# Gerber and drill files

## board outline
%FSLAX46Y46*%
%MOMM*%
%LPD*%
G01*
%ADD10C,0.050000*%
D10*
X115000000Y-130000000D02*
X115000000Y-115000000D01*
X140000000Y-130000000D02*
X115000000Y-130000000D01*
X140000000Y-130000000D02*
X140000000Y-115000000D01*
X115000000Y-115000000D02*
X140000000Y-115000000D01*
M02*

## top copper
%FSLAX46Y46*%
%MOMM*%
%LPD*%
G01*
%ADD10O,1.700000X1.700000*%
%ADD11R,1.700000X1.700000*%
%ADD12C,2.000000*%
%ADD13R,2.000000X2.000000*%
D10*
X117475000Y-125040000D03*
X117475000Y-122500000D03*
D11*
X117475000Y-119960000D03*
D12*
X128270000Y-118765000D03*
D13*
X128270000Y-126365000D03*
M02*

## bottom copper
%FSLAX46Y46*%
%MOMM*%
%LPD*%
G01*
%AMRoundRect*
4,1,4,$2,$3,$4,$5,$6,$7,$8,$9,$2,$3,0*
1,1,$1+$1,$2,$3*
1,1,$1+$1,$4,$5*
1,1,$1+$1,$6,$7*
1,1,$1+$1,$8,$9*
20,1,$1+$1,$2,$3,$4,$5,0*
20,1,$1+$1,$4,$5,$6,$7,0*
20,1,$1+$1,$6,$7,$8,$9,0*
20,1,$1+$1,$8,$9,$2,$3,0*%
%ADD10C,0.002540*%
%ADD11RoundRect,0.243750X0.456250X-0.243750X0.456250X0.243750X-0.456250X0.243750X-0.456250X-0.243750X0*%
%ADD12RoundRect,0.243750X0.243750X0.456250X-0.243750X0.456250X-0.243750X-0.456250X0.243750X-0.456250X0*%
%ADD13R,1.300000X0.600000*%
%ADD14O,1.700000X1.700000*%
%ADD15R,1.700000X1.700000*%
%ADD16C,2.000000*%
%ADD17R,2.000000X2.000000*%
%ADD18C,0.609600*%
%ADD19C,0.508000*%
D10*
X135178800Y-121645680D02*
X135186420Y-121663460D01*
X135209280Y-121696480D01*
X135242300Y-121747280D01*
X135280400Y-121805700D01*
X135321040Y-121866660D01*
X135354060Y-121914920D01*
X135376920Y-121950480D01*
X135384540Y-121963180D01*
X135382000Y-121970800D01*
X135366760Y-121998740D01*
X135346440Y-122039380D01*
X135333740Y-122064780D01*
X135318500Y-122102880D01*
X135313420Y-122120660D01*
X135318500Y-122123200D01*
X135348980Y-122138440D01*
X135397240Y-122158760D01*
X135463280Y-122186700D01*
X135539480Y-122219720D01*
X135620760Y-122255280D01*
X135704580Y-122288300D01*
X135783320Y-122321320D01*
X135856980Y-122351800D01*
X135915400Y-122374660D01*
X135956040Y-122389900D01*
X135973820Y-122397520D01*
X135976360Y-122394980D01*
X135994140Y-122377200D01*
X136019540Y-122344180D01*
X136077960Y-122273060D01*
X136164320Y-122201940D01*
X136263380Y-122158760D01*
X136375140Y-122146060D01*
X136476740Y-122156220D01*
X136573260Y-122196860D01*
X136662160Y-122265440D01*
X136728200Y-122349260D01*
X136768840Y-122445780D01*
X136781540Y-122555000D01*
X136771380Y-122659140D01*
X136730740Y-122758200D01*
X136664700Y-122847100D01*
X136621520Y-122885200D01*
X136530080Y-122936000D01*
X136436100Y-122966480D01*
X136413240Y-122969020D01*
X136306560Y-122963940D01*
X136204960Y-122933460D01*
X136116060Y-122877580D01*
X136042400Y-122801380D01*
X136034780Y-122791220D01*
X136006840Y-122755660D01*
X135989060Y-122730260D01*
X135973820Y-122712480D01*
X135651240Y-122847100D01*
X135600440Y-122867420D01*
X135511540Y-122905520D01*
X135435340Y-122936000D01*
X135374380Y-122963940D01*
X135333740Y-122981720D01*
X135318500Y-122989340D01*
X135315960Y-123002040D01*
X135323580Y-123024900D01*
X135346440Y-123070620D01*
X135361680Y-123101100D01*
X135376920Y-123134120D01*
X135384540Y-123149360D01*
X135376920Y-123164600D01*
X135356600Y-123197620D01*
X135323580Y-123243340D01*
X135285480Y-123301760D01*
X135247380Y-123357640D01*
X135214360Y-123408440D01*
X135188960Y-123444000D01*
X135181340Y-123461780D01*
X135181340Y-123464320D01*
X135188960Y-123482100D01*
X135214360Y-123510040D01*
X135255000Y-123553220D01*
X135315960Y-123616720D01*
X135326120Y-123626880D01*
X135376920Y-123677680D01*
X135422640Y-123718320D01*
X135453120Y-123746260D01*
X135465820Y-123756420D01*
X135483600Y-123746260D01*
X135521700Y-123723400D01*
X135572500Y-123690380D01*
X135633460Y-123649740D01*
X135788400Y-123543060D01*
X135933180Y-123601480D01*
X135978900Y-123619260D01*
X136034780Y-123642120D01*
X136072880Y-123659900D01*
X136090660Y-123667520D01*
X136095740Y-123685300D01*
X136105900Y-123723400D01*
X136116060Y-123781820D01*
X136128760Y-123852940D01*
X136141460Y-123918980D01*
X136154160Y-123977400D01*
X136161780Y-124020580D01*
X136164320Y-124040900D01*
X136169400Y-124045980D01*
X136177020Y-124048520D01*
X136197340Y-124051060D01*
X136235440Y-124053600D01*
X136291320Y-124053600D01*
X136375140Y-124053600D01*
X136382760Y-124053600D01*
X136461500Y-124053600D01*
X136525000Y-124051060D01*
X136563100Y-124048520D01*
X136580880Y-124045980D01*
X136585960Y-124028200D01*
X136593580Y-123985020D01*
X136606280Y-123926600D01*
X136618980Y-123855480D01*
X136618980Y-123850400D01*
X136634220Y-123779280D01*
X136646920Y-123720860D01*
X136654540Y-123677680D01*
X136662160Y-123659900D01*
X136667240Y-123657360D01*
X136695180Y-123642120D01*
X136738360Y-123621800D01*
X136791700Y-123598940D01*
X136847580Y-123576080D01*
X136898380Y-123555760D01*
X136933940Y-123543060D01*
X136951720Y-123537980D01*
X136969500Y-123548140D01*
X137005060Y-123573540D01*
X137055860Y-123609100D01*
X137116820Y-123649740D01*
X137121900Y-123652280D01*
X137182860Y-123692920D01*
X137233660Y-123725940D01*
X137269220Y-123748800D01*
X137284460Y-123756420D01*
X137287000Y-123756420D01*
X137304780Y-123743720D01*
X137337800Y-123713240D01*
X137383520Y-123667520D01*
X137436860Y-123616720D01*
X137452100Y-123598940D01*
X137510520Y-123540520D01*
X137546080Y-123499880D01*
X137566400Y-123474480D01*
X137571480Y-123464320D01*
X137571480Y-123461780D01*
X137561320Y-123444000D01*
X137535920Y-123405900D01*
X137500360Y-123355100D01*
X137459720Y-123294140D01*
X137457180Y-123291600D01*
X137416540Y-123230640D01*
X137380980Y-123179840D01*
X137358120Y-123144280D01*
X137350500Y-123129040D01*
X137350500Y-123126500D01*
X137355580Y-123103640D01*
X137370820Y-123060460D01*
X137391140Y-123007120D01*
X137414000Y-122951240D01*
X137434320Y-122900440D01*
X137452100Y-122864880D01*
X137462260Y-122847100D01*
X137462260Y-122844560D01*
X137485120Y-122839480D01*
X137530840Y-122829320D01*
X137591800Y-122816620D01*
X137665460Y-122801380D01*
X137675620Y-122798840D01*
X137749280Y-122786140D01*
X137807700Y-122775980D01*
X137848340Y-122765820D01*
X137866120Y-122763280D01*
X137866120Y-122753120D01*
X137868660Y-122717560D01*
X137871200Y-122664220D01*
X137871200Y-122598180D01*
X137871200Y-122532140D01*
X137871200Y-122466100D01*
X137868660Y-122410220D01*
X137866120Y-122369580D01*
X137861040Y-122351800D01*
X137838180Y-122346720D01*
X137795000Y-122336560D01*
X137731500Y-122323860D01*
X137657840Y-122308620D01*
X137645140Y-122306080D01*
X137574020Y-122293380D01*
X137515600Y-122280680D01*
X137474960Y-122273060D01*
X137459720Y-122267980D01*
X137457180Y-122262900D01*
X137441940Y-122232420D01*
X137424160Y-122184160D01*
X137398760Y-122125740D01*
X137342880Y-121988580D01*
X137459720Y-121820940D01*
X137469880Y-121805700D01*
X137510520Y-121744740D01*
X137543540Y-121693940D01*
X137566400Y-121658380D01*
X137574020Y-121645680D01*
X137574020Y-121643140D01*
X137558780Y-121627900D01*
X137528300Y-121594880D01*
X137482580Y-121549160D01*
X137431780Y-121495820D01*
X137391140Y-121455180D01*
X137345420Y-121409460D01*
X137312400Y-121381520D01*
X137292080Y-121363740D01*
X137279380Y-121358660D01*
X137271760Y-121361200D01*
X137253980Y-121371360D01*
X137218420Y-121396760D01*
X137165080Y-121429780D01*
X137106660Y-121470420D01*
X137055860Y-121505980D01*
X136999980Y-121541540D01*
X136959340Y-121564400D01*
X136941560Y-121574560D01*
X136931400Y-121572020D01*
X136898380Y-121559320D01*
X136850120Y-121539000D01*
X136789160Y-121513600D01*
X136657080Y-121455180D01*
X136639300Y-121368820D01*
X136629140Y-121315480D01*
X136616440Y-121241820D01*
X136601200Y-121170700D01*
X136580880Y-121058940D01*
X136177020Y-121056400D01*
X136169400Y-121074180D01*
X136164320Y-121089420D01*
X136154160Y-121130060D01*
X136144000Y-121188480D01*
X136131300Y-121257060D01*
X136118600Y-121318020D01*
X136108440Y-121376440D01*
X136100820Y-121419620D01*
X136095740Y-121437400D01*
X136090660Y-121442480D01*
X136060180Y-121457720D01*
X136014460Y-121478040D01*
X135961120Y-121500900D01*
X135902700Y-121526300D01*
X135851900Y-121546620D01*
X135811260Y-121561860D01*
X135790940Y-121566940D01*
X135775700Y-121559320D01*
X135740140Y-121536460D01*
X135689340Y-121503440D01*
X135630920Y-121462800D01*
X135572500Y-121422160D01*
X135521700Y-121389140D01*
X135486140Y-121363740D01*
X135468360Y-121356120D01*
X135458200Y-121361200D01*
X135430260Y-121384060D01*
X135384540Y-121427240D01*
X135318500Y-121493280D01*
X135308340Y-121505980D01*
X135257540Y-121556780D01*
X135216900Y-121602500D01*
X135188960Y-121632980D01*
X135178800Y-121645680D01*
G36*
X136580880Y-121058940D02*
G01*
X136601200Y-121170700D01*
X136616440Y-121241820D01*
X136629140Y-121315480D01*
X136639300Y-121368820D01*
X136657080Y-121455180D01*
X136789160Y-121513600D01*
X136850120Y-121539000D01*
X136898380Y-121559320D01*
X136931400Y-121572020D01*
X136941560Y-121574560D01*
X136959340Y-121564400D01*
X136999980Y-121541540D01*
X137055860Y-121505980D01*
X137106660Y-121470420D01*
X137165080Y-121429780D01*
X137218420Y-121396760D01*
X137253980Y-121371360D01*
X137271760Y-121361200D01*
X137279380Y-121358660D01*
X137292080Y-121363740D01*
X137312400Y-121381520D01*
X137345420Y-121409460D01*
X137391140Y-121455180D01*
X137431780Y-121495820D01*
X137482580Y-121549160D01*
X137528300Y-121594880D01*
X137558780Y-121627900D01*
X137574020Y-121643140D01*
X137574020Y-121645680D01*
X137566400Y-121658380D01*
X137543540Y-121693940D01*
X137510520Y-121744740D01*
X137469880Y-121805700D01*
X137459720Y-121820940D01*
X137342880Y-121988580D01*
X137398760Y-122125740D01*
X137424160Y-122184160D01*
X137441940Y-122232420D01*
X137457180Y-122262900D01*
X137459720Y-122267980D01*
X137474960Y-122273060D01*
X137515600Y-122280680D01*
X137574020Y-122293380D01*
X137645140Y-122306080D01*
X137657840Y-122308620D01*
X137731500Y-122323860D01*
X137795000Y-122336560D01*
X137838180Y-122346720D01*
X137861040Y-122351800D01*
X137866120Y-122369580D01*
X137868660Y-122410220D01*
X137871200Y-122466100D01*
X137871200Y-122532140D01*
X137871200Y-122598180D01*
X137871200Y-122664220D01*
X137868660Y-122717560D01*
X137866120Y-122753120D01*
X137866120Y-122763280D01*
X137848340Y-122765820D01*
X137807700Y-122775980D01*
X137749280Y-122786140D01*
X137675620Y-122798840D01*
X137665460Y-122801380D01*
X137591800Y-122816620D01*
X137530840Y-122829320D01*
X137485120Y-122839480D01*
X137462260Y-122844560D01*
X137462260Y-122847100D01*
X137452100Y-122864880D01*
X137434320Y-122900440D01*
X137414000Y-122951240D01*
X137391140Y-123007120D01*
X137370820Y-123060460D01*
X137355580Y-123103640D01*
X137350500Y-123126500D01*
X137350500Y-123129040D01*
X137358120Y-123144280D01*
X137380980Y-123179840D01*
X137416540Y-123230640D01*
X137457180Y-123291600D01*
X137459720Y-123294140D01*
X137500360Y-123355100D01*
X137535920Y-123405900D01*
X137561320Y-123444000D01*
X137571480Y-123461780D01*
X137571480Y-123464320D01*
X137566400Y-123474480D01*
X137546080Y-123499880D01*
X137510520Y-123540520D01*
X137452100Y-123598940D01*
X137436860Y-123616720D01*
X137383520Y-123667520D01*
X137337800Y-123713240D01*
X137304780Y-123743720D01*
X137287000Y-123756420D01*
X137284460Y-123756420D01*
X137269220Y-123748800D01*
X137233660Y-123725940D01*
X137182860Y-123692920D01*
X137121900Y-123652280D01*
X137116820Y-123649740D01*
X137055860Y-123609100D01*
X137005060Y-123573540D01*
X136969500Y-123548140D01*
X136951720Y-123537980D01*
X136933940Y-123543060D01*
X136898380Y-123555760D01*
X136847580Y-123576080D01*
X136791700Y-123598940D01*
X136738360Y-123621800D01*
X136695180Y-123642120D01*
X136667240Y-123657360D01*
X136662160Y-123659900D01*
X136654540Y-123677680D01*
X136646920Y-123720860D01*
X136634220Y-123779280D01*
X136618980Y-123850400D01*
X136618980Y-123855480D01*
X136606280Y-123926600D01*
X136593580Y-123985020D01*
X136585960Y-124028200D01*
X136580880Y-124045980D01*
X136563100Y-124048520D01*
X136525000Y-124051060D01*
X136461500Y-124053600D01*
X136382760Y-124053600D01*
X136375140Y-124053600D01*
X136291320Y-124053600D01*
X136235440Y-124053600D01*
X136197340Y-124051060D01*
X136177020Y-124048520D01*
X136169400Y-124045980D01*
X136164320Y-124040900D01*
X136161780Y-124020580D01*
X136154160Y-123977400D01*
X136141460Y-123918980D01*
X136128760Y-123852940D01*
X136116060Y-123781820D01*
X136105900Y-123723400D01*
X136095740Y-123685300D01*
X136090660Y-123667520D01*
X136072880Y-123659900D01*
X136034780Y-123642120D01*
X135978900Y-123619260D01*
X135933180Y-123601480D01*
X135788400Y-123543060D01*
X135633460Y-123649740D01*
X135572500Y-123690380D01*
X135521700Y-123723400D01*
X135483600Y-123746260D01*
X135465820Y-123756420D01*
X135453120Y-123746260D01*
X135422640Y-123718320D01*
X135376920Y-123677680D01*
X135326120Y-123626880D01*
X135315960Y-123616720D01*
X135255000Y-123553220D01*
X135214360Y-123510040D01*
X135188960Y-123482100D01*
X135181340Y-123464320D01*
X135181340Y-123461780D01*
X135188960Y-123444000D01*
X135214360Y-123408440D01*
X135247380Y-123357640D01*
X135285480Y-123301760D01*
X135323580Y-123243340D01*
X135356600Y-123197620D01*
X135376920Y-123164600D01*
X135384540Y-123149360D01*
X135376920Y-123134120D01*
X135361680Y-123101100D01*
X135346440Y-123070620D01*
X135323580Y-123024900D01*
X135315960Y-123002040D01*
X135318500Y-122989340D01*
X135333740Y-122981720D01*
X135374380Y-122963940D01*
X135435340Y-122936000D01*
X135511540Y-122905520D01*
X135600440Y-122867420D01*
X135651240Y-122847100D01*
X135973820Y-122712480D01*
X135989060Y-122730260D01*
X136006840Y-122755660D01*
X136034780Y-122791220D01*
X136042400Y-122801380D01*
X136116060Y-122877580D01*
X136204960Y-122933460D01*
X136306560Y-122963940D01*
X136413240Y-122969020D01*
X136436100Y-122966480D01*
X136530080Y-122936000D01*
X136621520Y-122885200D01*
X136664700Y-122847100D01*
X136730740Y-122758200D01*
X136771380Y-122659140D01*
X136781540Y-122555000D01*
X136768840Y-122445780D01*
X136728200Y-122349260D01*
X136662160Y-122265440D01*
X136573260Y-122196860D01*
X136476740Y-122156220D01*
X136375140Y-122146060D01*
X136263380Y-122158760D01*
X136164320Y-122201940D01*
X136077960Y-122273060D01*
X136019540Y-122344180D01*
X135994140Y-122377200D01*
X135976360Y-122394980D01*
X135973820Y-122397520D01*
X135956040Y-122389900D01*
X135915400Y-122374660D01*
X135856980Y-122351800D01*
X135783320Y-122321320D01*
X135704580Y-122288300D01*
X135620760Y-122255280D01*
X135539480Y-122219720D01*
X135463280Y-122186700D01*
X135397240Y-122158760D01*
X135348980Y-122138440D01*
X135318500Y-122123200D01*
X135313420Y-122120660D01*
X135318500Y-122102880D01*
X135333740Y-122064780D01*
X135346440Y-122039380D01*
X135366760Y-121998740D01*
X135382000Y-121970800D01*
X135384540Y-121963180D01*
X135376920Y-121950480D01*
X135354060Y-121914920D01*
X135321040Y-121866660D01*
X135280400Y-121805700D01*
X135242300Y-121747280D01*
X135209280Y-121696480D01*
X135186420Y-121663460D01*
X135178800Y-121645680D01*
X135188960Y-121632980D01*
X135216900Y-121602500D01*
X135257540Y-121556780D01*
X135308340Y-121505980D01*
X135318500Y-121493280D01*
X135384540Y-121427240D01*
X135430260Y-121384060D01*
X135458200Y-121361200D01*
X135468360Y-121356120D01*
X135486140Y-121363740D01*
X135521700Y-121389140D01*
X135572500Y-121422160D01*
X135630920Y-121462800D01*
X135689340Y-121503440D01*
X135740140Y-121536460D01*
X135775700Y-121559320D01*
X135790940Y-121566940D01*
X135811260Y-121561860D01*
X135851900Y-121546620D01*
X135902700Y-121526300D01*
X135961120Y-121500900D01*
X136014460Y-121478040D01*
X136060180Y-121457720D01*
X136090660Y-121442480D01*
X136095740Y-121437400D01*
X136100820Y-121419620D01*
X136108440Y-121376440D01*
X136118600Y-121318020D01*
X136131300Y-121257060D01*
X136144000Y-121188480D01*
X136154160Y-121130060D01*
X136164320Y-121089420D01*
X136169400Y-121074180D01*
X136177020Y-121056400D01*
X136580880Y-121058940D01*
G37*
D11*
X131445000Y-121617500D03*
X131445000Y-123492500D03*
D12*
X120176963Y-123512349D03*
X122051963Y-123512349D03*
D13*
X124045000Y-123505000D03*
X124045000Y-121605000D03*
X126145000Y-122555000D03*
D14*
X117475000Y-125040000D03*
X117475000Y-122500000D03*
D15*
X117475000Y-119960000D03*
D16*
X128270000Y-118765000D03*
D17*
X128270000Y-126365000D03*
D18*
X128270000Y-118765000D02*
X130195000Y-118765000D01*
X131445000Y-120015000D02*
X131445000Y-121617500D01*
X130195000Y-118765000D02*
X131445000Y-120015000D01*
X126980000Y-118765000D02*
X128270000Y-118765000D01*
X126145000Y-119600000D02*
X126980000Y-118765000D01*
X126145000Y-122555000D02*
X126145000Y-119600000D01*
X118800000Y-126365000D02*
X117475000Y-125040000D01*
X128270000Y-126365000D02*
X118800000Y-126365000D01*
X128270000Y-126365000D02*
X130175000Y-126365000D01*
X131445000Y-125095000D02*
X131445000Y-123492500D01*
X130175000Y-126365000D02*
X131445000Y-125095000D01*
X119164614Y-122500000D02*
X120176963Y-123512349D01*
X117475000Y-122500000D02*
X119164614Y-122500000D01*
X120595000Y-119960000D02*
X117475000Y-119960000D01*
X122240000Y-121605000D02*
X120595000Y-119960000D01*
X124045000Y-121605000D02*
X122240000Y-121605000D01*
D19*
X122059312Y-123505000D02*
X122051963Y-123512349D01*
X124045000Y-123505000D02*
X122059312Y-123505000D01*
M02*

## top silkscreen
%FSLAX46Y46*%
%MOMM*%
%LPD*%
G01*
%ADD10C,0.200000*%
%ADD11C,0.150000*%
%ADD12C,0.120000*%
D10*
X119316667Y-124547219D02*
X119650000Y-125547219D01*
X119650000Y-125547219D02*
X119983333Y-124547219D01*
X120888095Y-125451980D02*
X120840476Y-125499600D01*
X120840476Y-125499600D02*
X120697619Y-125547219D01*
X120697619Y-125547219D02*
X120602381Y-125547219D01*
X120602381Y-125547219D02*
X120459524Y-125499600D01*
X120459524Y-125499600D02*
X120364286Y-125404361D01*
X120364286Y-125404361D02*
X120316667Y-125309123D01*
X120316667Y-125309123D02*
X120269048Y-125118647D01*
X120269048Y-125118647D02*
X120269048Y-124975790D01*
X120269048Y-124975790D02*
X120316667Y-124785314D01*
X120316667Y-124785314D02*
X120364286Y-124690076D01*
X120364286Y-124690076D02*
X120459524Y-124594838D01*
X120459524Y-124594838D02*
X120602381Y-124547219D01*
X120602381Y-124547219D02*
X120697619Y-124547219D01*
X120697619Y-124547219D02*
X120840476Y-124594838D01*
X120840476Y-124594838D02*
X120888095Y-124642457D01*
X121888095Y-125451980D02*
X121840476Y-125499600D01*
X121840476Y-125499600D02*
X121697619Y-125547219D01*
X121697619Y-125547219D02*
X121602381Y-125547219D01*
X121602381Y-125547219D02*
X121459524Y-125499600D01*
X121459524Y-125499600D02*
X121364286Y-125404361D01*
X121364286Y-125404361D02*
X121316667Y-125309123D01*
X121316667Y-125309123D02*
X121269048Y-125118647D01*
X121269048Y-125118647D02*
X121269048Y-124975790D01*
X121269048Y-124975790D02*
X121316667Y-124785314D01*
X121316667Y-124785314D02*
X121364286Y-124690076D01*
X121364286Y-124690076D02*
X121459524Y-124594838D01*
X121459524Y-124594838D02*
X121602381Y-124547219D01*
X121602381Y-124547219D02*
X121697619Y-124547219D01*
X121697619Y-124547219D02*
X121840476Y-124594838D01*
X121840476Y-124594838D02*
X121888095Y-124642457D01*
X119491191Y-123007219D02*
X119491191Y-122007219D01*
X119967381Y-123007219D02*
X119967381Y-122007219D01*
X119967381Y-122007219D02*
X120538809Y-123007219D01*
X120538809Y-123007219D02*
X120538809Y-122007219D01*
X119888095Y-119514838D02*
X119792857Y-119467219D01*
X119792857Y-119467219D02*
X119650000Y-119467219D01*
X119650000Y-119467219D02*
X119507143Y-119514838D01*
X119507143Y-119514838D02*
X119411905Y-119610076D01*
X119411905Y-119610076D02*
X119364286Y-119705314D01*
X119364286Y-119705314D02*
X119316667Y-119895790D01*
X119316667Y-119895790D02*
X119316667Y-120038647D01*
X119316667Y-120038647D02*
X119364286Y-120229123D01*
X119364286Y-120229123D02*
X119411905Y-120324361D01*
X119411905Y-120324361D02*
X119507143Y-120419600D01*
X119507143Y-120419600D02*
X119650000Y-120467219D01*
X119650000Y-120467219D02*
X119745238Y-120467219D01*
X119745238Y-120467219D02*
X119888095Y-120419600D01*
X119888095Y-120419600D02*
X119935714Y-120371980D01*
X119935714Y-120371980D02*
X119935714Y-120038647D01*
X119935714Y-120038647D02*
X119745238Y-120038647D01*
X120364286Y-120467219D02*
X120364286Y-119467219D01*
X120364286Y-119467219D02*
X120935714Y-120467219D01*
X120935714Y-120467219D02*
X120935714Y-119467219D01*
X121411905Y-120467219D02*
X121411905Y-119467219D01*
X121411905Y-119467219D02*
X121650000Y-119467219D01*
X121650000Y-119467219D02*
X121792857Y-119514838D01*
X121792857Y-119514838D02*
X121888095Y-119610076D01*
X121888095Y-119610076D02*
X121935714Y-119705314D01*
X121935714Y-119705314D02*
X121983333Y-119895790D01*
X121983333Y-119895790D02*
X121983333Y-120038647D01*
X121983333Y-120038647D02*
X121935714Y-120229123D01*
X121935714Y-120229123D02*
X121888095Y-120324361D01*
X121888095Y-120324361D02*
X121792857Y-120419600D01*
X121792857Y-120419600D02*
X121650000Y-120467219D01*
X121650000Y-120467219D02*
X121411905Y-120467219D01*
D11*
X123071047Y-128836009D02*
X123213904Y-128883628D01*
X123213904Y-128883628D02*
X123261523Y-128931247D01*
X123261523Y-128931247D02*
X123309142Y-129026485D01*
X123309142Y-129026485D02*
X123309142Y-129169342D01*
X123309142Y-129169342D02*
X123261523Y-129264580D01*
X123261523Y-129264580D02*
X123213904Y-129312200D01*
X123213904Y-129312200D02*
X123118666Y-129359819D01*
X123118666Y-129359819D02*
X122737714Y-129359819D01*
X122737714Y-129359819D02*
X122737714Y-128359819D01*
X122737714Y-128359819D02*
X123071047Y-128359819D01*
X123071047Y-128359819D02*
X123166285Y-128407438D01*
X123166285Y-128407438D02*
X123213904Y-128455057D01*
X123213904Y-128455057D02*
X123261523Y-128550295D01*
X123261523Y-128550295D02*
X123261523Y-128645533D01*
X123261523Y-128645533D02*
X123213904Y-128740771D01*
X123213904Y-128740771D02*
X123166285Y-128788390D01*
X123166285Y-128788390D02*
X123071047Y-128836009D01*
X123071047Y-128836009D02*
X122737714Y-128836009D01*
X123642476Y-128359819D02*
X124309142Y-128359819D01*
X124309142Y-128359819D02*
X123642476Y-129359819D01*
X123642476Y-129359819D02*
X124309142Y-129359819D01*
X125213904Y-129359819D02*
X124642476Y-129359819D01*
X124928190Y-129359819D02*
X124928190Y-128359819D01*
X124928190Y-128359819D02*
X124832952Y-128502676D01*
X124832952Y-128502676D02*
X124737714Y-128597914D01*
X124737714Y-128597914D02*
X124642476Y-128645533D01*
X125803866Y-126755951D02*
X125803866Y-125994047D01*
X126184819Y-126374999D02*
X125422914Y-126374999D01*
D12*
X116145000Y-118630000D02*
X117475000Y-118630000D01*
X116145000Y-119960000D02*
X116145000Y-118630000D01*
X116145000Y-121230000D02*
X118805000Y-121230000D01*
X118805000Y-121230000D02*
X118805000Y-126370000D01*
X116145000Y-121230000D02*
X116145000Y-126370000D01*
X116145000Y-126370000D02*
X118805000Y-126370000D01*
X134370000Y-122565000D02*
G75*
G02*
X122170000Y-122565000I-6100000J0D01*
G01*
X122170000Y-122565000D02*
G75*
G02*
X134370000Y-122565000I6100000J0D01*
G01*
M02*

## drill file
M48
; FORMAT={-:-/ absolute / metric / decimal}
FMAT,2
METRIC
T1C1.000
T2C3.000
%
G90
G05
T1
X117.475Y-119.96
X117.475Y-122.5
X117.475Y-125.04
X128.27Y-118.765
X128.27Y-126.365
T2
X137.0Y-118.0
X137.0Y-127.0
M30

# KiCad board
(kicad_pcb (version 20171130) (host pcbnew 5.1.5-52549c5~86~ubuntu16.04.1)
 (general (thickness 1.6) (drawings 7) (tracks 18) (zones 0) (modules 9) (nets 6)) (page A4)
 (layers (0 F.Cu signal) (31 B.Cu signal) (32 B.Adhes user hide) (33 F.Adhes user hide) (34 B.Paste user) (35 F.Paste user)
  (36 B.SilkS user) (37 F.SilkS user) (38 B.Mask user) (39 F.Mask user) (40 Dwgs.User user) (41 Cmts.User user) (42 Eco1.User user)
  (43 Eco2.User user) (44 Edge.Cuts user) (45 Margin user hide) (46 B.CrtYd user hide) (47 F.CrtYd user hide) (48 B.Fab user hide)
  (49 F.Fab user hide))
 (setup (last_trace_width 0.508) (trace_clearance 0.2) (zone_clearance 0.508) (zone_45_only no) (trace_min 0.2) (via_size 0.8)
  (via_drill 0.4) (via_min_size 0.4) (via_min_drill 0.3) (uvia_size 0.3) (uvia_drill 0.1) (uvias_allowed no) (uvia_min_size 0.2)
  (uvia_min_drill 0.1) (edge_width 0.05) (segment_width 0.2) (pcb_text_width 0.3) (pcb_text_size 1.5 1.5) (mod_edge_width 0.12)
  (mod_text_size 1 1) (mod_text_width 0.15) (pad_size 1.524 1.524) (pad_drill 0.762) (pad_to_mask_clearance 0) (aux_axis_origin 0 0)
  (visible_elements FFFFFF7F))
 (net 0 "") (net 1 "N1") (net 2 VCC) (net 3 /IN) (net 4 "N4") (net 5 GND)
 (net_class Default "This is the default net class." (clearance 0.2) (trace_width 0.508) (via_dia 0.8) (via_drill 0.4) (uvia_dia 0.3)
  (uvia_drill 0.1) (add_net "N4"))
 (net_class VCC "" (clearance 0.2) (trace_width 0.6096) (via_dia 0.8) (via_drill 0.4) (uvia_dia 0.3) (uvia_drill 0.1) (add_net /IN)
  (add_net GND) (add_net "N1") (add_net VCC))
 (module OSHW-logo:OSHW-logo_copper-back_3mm (layer B.Cu) (at 136.525 122.555 90)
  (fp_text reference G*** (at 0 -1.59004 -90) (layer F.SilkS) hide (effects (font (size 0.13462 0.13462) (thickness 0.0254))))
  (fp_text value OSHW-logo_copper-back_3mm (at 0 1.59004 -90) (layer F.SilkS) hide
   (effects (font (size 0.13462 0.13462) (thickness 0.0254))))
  (fp_poly
   (pts (xy 0.90932 -1.3462) (xy 0.89154 -1.33858) (xy 0.85852 -1.31572) (xy 0.80772 -1.2827) (xy 0.7493 -1.2446) (xy 0.68834 -1.20396)
    (xy 0.64008 -1.17094) (xy 0.60452 -1.14808) (xy 0.59182 -1.14046) (xy 0.5842 -1.143) (xy 0.55626 -1.15824) (xy 0.51562 -1.17856)
    (xy 0.49022 -1.19126) (xy 0.45212 -1.2065) (xy 0.43434 -1.21158) (xy 0.4318 -1.2065) (xy 0.41656 -1.17602) (xy 0.39624 -1.12776)
    (xy 0.3683 -1.06172) (xy 0.33528 -0.98552) (xy 0.29972 -0.90424) (xy 0.2667 -0.82042) (xy 0.23368 -0.74168) (xy 0.2032 -0.66802)
    (xy 0.18034 -0.6096) (xy 0.1651 -0.56896) (xy 0.15748 -0.55118) (xy 0.16002 -0.54864) (xy 0.1778 -0.53086) (xy 0.21082 -0.50546)
    (xy 0.28194 -0.44704) (xy 0.35306 -0.36068) (xy 0.39624 -0.26162) (xy 0.40894 -0.14986) (xy 0.39878 -0.04826) (xy 0.35814 0.04826)
    (xy 0.28956 0.13716) (xy 0.20574 0.2032) (xy 0.10922 0.24384) (xy 0 0.25654) (xy -0.10414 0.24638) (xy -0.2032 0.20574)
    (xy -0.2921 0.1397) (xy -0.3302 0.09652) (xy -0.381 0.00508) (xy -0.41148 -0.0889) (xy -0.41402 -0.11176) (xy -0.40894 -0.21844)
    (xy -0.37846 -0.32004) (xy -0.32258 -0.40894) (xy -0.24638 -0.4826) (xy -0.23622 -0.49022) (xy -0.20066 -0.51816) (xy -0.17526 -0.53594)
    (xy -0.15748 -0.55118) (xy -0.2921 -0.87376) (xy -0.31242 -0.92456) (xy -0.35052 -1.01346) (xy -0.381 -1.08966) (xy -0.40894 -1.15062)
    (xy -0.42672 -1.19126) (xy -0.43434 -1.2065) (xy -0.44704 -1.20904) (xy -0.4699 -1.20142) (xy -0.51562 -1.17856) (xy -0.5461 -1.16332)
    (xy -0.57912 -1.14808) (xy -0.59436 -1.14046) (xy -0.6096 -1.14808) (xy -0.64262 -1.1684) (xy -0.68834 -1.20142) (xy -0.74676 -1.23952)
    (xy -0.80264 -1.27762) (xy -0.85344 -1.31064) (xy -0.889 -1.33604) (xy -0.90678 -1.34366) (xy -0.90932 -1.34366) (xy -0.9271 -1.33604)
    (xy -0.95504 -1.31064) (xy -0.99822 -1.27) (xy -1.06172 -1.20904) (xy -1.07188 -1.19888) (xy -1.12268 -1.14808) (xy -1.16332 -1.10236)
    (xy -1.19126 -1.07188) (xy -1.20142 -1.05918) (xy -1.19126 -1.0414) (xy -1.1684 -1.0033) (xy -1.13538 -0.9525) (xy -1.09474 -0.89154)
    (xy -0.98806 -0.7366) (xy -1.04648 -0.59182) (xy -1.06426 -0.5461) (xy -1.08712 -0.49022) (xy -1.1049 -0.45212) (xy -1.11252 -0.43434)
    (xy -1.1303 -0.42926) (xy -1.1684 -0.4191) (xy -1.22682 -0.40894) (xy -1.29794 -0.39624) (xy -1.36398 -0.38354) (xy -1.4224 -0.37084)
    (xy -1.46558 -0.36322) (xy -1.4859 -0.36068) (xy -1.49098 -0.3556) (xy -1.49352 -0.34798) (xy -1.49606 -0.32766) (xy -1.4986 -0.28956)
    (xy -1.4986 -0.23368) (xy -1.4986 -0.14986) (xy -1.4986 -0.14224) (xy -1.4986 -0.0635) (xy -1.49606 0) (xy -1.49352 0.0381)
    (xy -1.49098 0.05588) (xy -1.4732 0.06096) (xy -1.43002 0.06858) (xy -1.3716 0.08128) (xy -1.30048 0.09398) (xy -1.2954 0.09398)
    (xy -1.22428 0.10922) (xy -1.16586 0.12192) (xy -1.12268 0.12954) (xy -1.1049 0.13716) (xy -1.10236 0.14224) (xy -1.08712 0.17018)
    (xy -1.0668 0.21336) (xy -1.04394 0.2667) (xy -1.02108 0.32258) (xy -1.00076 0.37338) (xy -0.98806 0.40894) (xy -0.98298 0.42672)
    (xy -0.99314 0.4445) (xy -1.01854 0.48006) (xy -1.0541 0.53086) (xy -1.09474 0.59182) (xy -1.09728 0.5969) (xy -1.13792 0.65786)
    (xy -1.17094 0.70866) (xy -1.1938 0.74422) (xy -1.20142 0.75946) (xy -1.20142 0.762) (xy -1.18872 0.77978) (xy -1.15824 0.8128)
    (xy -1.11252 0.85852) (xy -1.06172 0.91186) (xy -1.04394 0.9271) (xy -0.98552 0.98552) (xy -0.94488 1.02108) (xy -0.91948 1.0414)
    (xy -0.90932 1.04648) (xy -0.90678 1.04648) (xy -0.889 1.03632) (xy -0.8509 1.01092) (xy -0.8001 0.97536) (xy -0.73914 0.93472)
    (xy -0.7366 0.93218) (xy -0.67564 0.89154) (xy -0.62484 0.85598) (xy -0.58928 0.83312) (xy -0.57404 0.8255) (xy -0.5715 0.8255)
    (xy -0.54864 0.83058) (xy -0.50546 0.84582) (xy -0.45212 0.86614) (xy -0.39624 0.889) (xy -0.34544 0.90932) (xy -0.30988 0.9271)
    (xy -0.2921 0.93726) (xy -0.28956 0.93726) (xy -0.28448 0.96012) (xy -0.27432 1.00584) (xy -0.26162 1.0668) (xy -0.24638 1.14046)
    (xy -0.24384 1.15062) (xy -0.23114 1.22428) (xy -0.22098 1.2827) (xy -0.21082 1.32334) (xy -0.20828 1.34112) (xy -0.19812 1.34112)
    (xy -0.16256 1.34366) (xy -0.10922 1.3462) (xy -0.04318 1.3462) (xy 0.02286 1.3462) (xy 0.0889 1.3462) (xy 0.14478 1.34366)
    (xy 0.18542 1.34112) (xy 0.2032 1.33604) (xy 0.20828 1.31318) (xy 0.21844 1.27) (xy 0.23114 1.2065) (xy 0.24638 1.13284)
    (xy 0.24892 1.12014) (xy 0.26162 1.04902) (xy 0.27432 0.9906) (xy 0.28194 0.94996) (xy 0.28702 0.93472) (xy 0.2921 0.93218)
    (xy 0.32258 0.91694) (xy 0.37084 0.89916) (xy 0.42926 0.87376) (xy 0.56642 0.81788) (xy 0.73406 0.93472) (xy 0.7493 0.94488)
    (xy 0.81026 0.98552) (xy 0.86106 1.01854) (xy 0.89662 1.0414) (xy 0.90932 1.04902) (xy 0.91186 1.04902) (xy 0.9271 1.03378)
    (xy 0.96012 1.0033) (xy 1.00584 0.95758) (xy 1.05918 0.90678) (xy 1.09982 0.86614) (xy 1.14554 0.82042) (xy 1.17348 0.7874)
    (xy 1.19126 0.76708) (xy 1.19634 0.75438) (xy 1.1938 0.74676) (xy 1.18364 0.72898) (xy 1.15824 0.69342) (xy 1.12522 0.64008)
    (xy 1.08458 0.58166) (xy 1.04902 0.53086) (xy 1.01346 0.47498) (xy 0.9906 0.43434) (xy 0.98044 0.41656) (xy 0.98298 0.4064)
    (xy 0.99568 0.37338) (xy 1.016 0.32512) (xy 1.0414 0.26416) (xy 1.09982 0.13208) (xy 1.18618 0.1143) (xy 1.23952 0.10414)
    (xy 1.31318 0.09144) (xy 1.3843 0.0762) (xy 1.49606 0.05588) (xy 1.4986 -0.34798) (xy 1.48082 -0.3556) (xy 1.46558 -0.36068)
    (xy 1.42494 -0.37084) (xy 1.36652 -0.381) (xy 1.29794 -0.3937) (xy 1.23698 -0.4064) (xy 1.17856 -0.41656) (xy 1.13538 -0.42418)
    (xy 1.1176 -0.42926) (xy 1.11252 -0.43434) (xy 1.09728 -0.46482) (xy 1.07696 -0.51054) (xy 1.0541 -0.56388) (xy 1.0287 -0.6223)
    (xy 1.00838 -0.6731) (xy 0.99314 -0.71374) (xy 0.98806 -0.73406) (xy 0.99568 -0.7493) (xy 1.01854 -0.78486) (xy 1.05156 -0.83566)
    (xy 1.0922 -0.89408) (xy 1.13284 -0.9525) (xy 1.16586 -1.0033) (xy 1.19126 -1.03886) (xy 1.19888 -1.05664) (xy 1.1938 -1.0668)
    (xy 1.17094 -1.09474) (xy 1.12776 -1.14046) (xy 1.06172 -1.2065) (xy 1.04902 -1.21666) (xy 0.99822 -1.26746) (xy 0.9525 -1.3081)
    (xy 0.92202 -1.33604) (xy 0.90932 -1.3462))
   (layer B.Cu) (width 0.00254)))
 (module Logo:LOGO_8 (layer B.Cu) (at 133.985 122.555 90)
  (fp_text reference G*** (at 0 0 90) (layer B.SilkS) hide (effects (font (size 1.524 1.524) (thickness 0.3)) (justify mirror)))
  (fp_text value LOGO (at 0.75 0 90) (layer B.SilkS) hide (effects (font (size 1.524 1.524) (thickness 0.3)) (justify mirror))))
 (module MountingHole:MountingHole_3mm (layer F.Cu) (at 137 118)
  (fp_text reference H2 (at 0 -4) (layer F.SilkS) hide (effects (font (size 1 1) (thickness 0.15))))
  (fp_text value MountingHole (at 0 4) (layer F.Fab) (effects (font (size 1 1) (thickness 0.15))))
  (pad 1 np_thru_hole circle (at 0 0) (size 3 3) (drill 3) (layers *.Cu *.Mask)))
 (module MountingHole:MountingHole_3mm (layer F.Cu) (at 137 127)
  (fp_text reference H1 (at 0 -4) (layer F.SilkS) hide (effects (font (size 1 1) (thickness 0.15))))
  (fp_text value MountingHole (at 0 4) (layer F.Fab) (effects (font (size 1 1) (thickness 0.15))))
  (pad 1 np_thru_hole circle (at 0 0) (size 3 3) (drill 3) (layers *.Cu *.Mask)))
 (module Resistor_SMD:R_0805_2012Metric (layer B.Cu) (at 131.445 122.555 90)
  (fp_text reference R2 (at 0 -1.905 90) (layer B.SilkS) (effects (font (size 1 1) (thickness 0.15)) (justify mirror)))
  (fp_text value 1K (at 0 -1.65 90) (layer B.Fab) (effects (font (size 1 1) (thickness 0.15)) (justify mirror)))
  (pad 2 smd roundrect (at 0.9375 0 90) (size 0.975 1.4) (layers B.Cu B.Paste B.Mask) (roundrect_rratio 0.25) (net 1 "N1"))
  (pad 1 smd roundrect (at -0.9375 0 90) (size 0.975 1.4) (layers B.Cu B.Paste B.Mask) (roundrect_rratio 0.25) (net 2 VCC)))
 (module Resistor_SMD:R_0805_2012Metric (layer B.Cu) (at 121.114463 123.512349 180)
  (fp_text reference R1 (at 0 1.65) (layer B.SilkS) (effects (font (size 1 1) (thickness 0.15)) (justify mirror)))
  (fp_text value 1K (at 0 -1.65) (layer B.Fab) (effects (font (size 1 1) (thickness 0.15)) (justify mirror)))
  (pad 2 smd roundrect (at 0.9375 0 180) (size 0.975 1.4) (layers B.Cu B.Paste B.Mask) (roundrect_rratio 0.25) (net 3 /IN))
  (pad 1 smd roundrect (at -0.9375 0 180) (size 0.975 1.4) (layers B.Cu B.Paste B.Mask) (roundrect_rratio 0.25) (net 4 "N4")))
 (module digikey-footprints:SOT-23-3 (layer B.Cu) (at 125.095 122.555)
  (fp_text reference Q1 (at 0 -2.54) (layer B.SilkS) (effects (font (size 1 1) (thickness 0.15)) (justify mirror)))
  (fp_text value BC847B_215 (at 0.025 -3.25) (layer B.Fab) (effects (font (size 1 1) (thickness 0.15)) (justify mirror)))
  (pad 1 smd rect (at -1.05 0.95) (size 1.3 0.6) (layers B.Cu B.Paste B.Mask) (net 4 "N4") (solder_mask_margin 0.07))
  (pad 2 smd rect (at -1.05 -0.95) (size 1.3 0.6) (layers B.Cu B.Paste B.Mask) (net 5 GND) (solder_mask_margin 0.07))
  (pad 3 smd rect (at 1.05 0) (size 1.3 0.6) (layers B.Cu B.Paste B.Mask) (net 1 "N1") (solder_mask_margin 0.07)))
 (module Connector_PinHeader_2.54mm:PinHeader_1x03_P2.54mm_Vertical (layer F.Cu) (at 117.475 119.96)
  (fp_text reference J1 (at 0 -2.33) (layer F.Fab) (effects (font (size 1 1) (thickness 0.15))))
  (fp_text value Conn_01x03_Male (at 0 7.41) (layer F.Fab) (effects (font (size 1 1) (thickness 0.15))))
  (fp_line (start -1.33 -1.33) (end 0 -1.33) (layer F.SilkS) (width 0.12))
  (fp_line (start -1.33 0) (end -1.33 -1.33) (layer F.SilkS) (width 0.12))
  (fp_line (start -1.33 1.27) (end 1.33 1.27) (layer F.SilkS) (width 0.12))
  (fp_line (start 1.33 1.27) (end 1.33 6.41) (layer F.SilkS) (width 0.12))
  (fp_line (start -1.33 1.27) (end -1.33 6.41) (layer F.SilkS) (width 0.12))
  (fp_line (start -1.33 6.41) (end 1.33 6.41) (layer F.SilkS) (width 0.12))
  (pad 3 thru_hole oval (at 0 5.08) (size 1.7 1.7) (drill 1) (layers *.Cu *.Mask) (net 2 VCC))
  (pad 2 thru_hole oval (at 0 2.54) (size 1.7 1.7) (drill 1) (layers *.Cu *.Mask) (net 3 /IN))
  (pad 1 thru_hole rect (at 0 0) (size 1.7 1.7) (drill 1) (layers *.Cu *.Mask) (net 5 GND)))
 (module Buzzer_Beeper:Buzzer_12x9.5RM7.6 (layer F.Cu) (at 128.27 126.365 90)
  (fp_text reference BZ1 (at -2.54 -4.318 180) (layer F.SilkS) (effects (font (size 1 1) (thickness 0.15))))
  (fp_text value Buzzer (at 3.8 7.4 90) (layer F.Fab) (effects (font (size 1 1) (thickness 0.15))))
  (fp_circle (center 3.8 0) (end 9.9 0) (layer F.SilkS) (width 0.12))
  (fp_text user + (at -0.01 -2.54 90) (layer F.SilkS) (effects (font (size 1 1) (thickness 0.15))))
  (pad 2 thru_hole circle (at 7.6 0 90) (size 2 2) (drill 1) (layers *.Cu *.Mask) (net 1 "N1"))
  (pad 1 thru_hole rect (at 0 0 90) (size 2 2) (drill 1) (layers *.Cu *.Mask) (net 2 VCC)))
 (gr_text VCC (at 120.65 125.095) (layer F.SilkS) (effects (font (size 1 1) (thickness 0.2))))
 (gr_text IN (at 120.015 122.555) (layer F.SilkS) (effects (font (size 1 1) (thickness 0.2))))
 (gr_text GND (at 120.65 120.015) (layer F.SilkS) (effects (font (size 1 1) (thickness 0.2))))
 (gr_line (start 115 130) (end 115 115) (layer Edge.Cuts) (width 0.05))
 (gr_line (start 140 130) (end 115 130) (layer Edge.Cuts) (width 0.05))
 (gr_line (start 140 130) (end 140 115) (layer Edge.Cuts) (width 0.05))
 (gr_line (start 115 115) (end 140 115) (layer Edge.Cuts) (width 0.05))
 (segment (start 128.27 118.765) (end 130.195 118.765) (width 0.6096) (layer B.Cu) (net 1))
 (segment (start 131.445 120.015) (end 131.445 121.6175) (width 0.6096) (layer B.Cu) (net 1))
 (segment (start 130.195 118.765) (end 131.445 120.015) (width 0.6096) (layer B.Cu) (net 1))
 (segment (start 126.98 118.765) (end 128.27 118.765) (width 0.6096) (layer B.Cu) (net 1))
 (segment (start 126.145 119.6) (end 126.98 118.765) (width 0.6096) (layer B.Cu) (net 1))
 (segment (start 126.145 122.555) (end 126.145 119.6) (width 0.6096) (layer B.Cu) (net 1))
 (segment (start 118.8 126.365) (end 117.475 125.04) (width 0.6096) (layer B.Cu) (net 2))
 (segment (start 128.27 126.365) (end 118.8 126.365) (width 0.6096) (layer B.Cu) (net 2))
 (segment (start 128.27 126.365) (end 130.175 126.365) (width 0.6096) (layer B.Cu) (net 2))
 (segment (start 131.445 125.095) (end 131.445 123.4925) (width 0.6096) (layer B.Cu) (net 2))
 (segment (start 130.175 126.365) (end 131.445 125.095) (width 0.6096) (layer B.Cu) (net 2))
 (segment (start 119.164614 122.5) (end 120.176963 123.512349) (width 0.6096) (layer B.Cu) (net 3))
 (segment (start 117.475 122.5) (end 119.164614 122.5) (width 0.6096) (layer B.Cu) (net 3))
 (segment (start 120.595 119.96) (end 117.475 119.96) (width 0.6096) (layer B.Cu) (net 5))
 (segment (start 122.24 121.605) (end 120.595 119.96) (width 0.6096) (layer B.Cu) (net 5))
 (segment (start 124.045 121.605) (end 122.24 121.605) (width 0.6096) (layer B.Cu) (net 5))
 (segment (start 122.059312 123.505) (end 122.051963 123.512349) (width 0.508) (layer B.Cu) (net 4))
 (segment (start 124.045 123.505) (end 122.059312 123.505) (width 0.508) (layer B.Cu) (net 4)))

